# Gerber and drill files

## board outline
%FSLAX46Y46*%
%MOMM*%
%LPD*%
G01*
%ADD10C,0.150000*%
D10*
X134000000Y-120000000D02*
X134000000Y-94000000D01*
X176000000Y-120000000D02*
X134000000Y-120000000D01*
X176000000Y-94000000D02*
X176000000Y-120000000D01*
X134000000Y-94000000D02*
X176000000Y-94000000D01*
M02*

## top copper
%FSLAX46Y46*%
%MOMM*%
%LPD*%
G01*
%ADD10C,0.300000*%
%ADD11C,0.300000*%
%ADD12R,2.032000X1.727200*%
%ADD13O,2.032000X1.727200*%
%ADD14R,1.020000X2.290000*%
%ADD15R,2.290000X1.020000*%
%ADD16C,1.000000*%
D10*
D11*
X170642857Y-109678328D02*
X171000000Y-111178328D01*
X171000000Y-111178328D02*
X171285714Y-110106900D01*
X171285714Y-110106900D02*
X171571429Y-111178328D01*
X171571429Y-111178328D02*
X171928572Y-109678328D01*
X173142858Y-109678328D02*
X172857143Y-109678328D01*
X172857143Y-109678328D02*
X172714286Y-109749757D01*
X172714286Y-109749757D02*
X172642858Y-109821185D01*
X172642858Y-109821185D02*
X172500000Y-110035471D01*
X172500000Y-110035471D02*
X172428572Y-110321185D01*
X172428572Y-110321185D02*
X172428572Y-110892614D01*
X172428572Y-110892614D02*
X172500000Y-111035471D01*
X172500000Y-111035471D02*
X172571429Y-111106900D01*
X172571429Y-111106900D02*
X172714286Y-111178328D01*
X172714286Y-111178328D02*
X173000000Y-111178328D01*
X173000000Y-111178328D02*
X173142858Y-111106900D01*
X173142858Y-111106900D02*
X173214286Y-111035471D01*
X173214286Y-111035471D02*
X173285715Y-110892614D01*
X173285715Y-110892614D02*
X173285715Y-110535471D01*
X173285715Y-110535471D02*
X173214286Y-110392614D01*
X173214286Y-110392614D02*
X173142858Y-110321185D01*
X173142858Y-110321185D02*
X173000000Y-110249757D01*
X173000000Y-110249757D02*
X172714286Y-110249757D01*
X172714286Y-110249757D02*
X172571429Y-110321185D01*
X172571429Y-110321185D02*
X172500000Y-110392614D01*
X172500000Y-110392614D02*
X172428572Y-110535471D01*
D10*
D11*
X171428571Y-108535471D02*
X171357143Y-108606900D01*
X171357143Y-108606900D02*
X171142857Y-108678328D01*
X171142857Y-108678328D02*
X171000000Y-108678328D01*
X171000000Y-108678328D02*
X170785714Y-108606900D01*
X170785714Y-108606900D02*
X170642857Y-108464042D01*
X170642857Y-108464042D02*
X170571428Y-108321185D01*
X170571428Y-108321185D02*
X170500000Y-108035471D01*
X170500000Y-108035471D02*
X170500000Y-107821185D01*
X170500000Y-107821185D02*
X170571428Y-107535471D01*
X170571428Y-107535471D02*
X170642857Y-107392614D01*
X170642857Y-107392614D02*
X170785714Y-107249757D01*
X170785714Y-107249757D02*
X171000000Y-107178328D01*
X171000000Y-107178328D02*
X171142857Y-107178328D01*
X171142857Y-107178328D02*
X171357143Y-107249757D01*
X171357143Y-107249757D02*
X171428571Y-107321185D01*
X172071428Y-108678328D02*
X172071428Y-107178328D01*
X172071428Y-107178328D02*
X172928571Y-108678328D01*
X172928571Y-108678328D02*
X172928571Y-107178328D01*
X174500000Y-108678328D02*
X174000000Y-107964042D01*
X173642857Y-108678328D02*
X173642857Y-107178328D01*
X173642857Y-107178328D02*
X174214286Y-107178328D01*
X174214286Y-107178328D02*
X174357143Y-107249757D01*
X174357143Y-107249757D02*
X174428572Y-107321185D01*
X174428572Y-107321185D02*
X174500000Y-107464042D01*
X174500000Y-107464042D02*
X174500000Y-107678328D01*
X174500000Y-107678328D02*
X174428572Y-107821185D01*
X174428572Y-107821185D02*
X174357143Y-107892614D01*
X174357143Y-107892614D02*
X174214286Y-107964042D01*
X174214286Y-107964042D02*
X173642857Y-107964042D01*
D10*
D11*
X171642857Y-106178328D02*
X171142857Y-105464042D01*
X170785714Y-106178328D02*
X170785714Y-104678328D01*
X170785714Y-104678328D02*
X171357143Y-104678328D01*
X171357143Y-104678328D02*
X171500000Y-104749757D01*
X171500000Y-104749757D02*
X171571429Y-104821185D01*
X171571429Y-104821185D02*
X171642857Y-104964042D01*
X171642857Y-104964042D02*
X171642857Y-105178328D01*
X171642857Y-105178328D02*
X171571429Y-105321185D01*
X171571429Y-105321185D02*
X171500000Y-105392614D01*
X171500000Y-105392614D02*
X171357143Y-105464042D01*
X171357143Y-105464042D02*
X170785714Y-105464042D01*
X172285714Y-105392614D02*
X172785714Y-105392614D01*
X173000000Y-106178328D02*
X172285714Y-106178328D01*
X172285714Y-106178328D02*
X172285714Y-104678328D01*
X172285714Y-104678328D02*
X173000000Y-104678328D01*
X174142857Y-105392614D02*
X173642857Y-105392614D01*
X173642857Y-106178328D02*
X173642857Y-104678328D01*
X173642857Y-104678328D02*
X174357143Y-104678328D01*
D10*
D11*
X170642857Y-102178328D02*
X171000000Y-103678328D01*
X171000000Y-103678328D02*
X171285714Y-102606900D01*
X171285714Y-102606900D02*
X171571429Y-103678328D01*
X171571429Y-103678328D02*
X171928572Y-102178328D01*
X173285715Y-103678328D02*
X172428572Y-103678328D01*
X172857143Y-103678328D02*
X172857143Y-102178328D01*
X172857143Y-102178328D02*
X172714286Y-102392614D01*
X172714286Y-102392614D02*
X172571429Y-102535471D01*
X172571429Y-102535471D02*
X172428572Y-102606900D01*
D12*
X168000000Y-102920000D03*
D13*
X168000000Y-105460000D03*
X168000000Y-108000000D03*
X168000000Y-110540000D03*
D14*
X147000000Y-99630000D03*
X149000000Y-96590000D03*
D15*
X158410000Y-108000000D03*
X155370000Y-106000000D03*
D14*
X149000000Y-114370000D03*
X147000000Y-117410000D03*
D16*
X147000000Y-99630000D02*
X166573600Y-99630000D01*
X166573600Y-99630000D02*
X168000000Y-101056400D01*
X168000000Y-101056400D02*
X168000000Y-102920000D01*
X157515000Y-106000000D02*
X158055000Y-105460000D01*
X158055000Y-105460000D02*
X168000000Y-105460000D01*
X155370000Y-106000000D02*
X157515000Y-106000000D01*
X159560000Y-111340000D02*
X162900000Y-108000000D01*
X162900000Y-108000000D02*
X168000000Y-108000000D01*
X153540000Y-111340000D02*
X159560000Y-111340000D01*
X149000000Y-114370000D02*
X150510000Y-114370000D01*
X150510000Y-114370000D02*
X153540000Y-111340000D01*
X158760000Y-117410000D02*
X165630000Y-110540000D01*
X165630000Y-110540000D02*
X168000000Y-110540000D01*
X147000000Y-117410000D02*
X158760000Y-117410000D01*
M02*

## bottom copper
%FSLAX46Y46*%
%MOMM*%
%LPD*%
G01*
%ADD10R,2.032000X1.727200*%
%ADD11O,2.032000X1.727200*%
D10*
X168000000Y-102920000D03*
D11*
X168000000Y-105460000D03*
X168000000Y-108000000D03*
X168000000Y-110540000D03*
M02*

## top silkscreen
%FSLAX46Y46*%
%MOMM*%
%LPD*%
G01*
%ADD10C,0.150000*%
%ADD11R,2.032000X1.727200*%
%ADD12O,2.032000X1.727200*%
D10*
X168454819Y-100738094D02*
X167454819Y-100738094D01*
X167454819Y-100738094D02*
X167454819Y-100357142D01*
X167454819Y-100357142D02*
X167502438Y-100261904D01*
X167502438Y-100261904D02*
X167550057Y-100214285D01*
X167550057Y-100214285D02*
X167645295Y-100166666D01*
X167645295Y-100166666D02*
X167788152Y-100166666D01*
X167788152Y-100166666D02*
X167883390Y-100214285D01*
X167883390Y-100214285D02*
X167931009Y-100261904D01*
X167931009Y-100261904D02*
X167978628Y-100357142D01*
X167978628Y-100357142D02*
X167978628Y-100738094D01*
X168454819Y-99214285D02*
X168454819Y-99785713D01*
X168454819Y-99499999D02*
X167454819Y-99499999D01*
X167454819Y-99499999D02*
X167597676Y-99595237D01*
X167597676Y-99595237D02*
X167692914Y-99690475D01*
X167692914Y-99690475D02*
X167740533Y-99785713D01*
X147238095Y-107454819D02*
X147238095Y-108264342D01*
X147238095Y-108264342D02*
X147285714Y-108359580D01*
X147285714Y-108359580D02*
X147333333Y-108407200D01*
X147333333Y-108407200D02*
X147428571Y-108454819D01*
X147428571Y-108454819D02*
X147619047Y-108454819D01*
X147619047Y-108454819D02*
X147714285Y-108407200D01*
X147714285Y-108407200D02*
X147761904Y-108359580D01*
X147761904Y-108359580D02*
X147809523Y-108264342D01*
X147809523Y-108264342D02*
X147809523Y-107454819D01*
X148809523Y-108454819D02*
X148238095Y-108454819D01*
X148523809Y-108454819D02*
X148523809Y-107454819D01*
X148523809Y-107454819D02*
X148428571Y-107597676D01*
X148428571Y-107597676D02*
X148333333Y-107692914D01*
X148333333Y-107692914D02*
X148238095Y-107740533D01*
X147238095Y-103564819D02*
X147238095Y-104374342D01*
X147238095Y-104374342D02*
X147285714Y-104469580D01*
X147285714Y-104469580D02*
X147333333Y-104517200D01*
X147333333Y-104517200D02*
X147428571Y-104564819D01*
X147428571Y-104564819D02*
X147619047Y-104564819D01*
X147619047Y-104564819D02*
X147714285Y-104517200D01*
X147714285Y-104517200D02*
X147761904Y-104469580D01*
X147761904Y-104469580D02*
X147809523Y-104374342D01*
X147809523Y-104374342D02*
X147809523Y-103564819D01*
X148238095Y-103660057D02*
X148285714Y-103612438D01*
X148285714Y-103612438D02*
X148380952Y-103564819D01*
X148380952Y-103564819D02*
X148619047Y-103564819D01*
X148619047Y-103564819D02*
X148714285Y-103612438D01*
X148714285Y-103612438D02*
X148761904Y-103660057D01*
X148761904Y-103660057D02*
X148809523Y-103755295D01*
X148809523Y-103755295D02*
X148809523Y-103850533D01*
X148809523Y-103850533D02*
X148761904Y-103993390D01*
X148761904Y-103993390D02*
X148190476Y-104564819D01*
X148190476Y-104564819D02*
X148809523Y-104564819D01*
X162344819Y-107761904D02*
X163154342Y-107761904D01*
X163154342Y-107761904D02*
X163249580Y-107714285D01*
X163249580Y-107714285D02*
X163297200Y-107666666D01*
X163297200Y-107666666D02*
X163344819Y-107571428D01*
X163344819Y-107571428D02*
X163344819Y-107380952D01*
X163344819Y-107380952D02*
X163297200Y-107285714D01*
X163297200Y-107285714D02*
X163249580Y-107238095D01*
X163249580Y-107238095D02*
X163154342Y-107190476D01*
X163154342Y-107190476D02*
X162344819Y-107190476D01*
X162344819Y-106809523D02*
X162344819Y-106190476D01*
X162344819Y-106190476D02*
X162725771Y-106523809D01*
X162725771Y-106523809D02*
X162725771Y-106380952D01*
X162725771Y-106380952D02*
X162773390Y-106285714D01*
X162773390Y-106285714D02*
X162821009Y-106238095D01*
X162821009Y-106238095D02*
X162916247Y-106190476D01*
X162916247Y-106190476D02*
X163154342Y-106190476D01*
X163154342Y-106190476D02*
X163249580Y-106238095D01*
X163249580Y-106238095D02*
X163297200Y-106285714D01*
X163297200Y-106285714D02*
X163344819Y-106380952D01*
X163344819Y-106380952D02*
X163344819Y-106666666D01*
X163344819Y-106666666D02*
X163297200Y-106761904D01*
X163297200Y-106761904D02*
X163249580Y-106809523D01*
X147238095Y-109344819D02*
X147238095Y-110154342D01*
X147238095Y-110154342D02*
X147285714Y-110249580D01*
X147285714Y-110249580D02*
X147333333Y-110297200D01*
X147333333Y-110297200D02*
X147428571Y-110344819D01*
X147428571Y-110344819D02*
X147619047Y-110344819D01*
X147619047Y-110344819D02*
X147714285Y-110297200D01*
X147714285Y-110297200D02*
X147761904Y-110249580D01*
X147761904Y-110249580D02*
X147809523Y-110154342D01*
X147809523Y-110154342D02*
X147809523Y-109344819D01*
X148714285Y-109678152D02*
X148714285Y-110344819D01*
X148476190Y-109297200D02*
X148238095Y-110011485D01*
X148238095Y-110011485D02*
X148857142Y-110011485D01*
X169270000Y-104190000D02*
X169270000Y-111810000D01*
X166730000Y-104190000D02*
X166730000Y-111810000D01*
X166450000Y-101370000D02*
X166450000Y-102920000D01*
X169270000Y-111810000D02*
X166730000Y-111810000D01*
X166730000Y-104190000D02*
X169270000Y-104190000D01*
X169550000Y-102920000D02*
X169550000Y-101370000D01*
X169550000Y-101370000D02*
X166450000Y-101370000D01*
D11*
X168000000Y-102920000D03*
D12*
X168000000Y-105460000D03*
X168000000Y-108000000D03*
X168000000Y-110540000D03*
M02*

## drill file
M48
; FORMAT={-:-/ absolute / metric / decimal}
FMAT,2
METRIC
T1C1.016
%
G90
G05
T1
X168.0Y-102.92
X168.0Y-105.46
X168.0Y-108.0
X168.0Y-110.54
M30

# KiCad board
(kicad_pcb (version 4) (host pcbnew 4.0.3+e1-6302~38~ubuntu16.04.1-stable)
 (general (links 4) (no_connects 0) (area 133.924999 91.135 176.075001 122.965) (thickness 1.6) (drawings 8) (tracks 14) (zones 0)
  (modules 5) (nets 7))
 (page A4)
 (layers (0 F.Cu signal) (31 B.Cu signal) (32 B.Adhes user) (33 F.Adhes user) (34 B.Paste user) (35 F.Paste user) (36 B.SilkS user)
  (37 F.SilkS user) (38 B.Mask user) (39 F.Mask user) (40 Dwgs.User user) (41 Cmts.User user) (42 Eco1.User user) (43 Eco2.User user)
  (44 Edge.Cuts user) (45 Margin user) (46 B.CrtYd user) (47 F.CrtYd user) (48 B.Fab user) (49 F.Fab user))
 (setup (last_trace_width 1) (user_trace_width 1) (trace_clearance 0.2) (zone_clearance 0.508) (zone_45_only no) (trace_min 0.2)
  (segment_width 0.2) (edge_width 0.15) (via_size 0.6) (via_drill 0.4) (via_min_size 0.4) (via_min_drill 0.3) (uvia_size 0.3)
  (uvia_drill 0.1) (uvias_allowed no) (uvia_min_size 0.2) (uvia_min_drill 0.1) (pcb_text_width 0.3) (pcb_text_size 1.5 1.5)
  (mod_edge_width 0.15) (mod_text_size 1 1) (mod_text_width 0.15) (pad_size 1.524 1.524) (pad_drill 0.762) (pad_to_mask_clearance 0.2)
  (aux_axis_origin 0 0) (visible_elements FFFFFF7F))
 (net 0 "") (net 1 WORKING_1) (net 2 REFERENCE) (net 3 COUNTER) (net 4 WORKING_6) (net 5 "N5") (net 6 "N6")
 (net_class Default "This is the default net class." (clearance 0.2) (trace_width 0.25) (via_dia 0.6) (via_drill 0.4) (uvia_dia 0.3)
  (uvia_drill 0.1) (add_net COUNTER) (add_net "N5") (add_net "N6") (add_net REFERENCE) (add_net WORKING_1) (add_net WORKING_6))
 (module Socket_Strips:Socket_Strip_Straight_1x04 (layer F.Cu) (at 168 102.92 270)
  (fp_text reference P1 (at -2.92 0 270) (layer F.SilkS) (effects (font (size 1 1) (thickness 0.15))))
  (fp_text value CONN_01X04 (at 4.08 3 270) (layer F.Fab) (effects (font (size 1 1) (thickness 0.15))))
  (fp_line (start 1.27 -1.27) (end 8.89 -1.27) (layer F.SilkS) (width 0.15))
  (fp_line (start 1.27 1.27) (end 8.89 1.27) (layer F.SilkS) (width 0.15))
  (fp_line (start -1.55 1.55) (end 0 1.55) (layer F.SilkS) (width 0.15))
  (fp_line (start 8.89 -1.27) (end 8.89 1.27) (layer F.SilkS) (width 0.15))
  (fp_line (start 1.27 1.27) (end 1.27 -1.27) (layer F.SilkS) (width 0.15))
  (fp_line (start 0 -1.55) (end -1.55 -1.55) (layer F.SilkS) (width 0.15))
  (fp_line (start -1.55 -1.55) (end -1.55 1.55) (layer F.SilkS) (width 0.15))
  (pad 1 thru_hole rect (at 0 0 270) (size 1.7272 2.032) (drill 1.016) (layers *.Cu *.Mask F.SilkS) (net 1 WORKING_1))
  (pad 2 thru_hole oval (at 2.54 0 270) (size 1.7272 2.032) (drill 1.016) (layers *.Cu *.Mask F.SilkS) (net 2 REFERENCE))
  (pad 3 thru_hole oval (at 5.08 0 270) (size 1.7272 2.032) (drill 1.016) (layers *.Cu *.Mask F.SilkS) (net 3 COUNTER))
  (pad 4 thru_hole oval (at 7.62 0 270) (size 1.7272 2.032) (drill 1.016) (layers *.Cu *.Mask F.SilkS) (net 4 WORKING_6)))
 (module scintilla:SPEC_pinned (layer F.Cu) (at 148 107)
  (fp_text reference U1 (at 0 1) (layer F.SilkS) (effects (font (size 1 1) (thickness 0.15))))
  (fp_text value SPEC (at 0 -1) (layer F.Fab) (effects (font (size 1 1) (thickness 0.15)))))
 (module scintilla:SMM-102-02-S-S (layer F.Cu) (at 148 98.11)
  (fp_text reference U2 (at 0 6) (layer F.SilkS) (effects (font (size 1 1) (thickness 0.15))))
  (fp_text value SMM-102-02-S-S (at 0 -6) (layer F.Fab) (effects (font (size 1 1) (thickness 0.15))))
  (pad 1 smd rect (at -1 1.52) (size 1.02 2.29) (layers F.Cu F.Paste F.Mask) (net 1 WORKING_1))
  (pad 2 smd rect (at 1 -1.52) (size 1.02 2.29) (layers F.Cu F.Paste F.Mask) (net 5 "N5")))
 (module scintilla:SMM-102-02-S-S (layer F.Cu) (at 156.89 107 90)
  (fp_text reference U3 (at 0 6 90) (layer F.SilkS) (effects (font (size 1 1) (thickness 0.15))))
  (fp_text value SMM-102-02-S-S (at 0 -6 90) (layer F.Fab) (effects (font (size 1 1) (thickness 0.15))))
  (pad 1 smd rect (at -1 1.52 90) (size 1.02 2.29) (layers F.Cu F.Paste F.Mask) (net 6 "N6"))
  (pad 2 smd rect (at 1 -1.52 90) (size 1.02 2.29) (layers F.Cu F.Paste F.Mask) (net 2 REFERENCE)))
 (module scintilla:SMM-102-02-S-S (layer F.Cu) (at 148 115.89 180)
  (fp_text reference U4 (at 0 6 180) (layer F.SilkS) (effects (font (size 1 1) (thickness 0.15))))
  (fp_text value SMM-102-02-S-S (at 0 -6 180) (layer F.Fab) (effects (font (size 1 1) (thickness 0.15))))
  (pad 1 smd rect (at -1 1.52 180) (size 1.02 2.29) (layers F.Cu F.Paste F.Mask) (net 3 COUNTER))
  (pad 2 smd rect (at 1 -1.52 180) (size 1.02 2.29) (layers F.Cu F.Paste F.Mask) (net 4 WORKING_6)))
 (gr_line (start 134 120) (end 134 94) (layer Edge.Cuts) (width 0.15))
 (gr_line (start 176 120) (end 134 120) (layer Edge.Cuts) (width 0.15))
 (gr_line (start 176 94) (end 176 120) (layer Edge.Cuts) (width 0.15))
 (gr_line (start 134 94) (end 176 94) (layer Edge.Cuts) (width 0.15))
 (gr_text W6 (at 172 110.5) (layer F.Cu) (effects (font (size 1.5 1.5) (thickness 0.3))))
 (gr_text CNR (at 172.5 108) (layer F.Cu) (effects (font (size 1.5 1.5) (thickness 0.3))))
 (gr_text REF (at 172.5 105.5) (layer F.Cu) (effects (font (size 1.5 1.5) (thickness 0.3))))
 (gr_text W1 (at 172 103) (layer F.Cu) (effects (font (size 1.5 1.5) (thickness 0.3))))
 (segment (start 147 99.63) (end 166.5736 99.63) (width 1) (layer F.Cu) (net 1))
 (segment (start 166.5736 99.63) (end 168 101.0564) (width 1) (layer F.Cu) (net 1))
 (segment (start 168 101.0564) (end 168 102.92) (width 1) (layer F.Cu) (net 1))
 (segment (start 157.515 106) (end 158.055 105.46) (width 1) (layer F.Cu) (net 2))
 (segment (start 158.055 105.46) (end 168 105.46) (width 1) (layer F.Cu) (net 2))
 (segment (start 155.37 106) (end 157.515 106) (width 1) (layer F.Cu) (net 2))
 (segment (start 159.56 111.34) (end 162.9 108) (width 1) (layer F.Cu) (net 3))
 (segment (start 162.9 108) (end 168 108) (width 1) (layer F.Cu) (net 3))
 (segment (start 153.54 111.34) (end 159.56 111.34) (width 1) (layer F.Cu) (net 3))
 (segment (start 149 114.37) (end 150.51 114.37) (width 1) (layer F.Cu) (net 3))
 (segment (start 150.51 114.37) (end 153.54 111.34) (width 1) (layer F.Cu) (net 3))
 (segment (start 158.76 117.41) (end 165.63 110.54) (width 1) (layer F.Cu) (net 4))
 (segment (start 165.63 110.54) (end 168 110.54) (width 1) (layer F.Cu) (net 4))
 (segment (start 147 117.41) (end 158.76 117.41) (width 1) (layer F.Cu) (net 4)))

